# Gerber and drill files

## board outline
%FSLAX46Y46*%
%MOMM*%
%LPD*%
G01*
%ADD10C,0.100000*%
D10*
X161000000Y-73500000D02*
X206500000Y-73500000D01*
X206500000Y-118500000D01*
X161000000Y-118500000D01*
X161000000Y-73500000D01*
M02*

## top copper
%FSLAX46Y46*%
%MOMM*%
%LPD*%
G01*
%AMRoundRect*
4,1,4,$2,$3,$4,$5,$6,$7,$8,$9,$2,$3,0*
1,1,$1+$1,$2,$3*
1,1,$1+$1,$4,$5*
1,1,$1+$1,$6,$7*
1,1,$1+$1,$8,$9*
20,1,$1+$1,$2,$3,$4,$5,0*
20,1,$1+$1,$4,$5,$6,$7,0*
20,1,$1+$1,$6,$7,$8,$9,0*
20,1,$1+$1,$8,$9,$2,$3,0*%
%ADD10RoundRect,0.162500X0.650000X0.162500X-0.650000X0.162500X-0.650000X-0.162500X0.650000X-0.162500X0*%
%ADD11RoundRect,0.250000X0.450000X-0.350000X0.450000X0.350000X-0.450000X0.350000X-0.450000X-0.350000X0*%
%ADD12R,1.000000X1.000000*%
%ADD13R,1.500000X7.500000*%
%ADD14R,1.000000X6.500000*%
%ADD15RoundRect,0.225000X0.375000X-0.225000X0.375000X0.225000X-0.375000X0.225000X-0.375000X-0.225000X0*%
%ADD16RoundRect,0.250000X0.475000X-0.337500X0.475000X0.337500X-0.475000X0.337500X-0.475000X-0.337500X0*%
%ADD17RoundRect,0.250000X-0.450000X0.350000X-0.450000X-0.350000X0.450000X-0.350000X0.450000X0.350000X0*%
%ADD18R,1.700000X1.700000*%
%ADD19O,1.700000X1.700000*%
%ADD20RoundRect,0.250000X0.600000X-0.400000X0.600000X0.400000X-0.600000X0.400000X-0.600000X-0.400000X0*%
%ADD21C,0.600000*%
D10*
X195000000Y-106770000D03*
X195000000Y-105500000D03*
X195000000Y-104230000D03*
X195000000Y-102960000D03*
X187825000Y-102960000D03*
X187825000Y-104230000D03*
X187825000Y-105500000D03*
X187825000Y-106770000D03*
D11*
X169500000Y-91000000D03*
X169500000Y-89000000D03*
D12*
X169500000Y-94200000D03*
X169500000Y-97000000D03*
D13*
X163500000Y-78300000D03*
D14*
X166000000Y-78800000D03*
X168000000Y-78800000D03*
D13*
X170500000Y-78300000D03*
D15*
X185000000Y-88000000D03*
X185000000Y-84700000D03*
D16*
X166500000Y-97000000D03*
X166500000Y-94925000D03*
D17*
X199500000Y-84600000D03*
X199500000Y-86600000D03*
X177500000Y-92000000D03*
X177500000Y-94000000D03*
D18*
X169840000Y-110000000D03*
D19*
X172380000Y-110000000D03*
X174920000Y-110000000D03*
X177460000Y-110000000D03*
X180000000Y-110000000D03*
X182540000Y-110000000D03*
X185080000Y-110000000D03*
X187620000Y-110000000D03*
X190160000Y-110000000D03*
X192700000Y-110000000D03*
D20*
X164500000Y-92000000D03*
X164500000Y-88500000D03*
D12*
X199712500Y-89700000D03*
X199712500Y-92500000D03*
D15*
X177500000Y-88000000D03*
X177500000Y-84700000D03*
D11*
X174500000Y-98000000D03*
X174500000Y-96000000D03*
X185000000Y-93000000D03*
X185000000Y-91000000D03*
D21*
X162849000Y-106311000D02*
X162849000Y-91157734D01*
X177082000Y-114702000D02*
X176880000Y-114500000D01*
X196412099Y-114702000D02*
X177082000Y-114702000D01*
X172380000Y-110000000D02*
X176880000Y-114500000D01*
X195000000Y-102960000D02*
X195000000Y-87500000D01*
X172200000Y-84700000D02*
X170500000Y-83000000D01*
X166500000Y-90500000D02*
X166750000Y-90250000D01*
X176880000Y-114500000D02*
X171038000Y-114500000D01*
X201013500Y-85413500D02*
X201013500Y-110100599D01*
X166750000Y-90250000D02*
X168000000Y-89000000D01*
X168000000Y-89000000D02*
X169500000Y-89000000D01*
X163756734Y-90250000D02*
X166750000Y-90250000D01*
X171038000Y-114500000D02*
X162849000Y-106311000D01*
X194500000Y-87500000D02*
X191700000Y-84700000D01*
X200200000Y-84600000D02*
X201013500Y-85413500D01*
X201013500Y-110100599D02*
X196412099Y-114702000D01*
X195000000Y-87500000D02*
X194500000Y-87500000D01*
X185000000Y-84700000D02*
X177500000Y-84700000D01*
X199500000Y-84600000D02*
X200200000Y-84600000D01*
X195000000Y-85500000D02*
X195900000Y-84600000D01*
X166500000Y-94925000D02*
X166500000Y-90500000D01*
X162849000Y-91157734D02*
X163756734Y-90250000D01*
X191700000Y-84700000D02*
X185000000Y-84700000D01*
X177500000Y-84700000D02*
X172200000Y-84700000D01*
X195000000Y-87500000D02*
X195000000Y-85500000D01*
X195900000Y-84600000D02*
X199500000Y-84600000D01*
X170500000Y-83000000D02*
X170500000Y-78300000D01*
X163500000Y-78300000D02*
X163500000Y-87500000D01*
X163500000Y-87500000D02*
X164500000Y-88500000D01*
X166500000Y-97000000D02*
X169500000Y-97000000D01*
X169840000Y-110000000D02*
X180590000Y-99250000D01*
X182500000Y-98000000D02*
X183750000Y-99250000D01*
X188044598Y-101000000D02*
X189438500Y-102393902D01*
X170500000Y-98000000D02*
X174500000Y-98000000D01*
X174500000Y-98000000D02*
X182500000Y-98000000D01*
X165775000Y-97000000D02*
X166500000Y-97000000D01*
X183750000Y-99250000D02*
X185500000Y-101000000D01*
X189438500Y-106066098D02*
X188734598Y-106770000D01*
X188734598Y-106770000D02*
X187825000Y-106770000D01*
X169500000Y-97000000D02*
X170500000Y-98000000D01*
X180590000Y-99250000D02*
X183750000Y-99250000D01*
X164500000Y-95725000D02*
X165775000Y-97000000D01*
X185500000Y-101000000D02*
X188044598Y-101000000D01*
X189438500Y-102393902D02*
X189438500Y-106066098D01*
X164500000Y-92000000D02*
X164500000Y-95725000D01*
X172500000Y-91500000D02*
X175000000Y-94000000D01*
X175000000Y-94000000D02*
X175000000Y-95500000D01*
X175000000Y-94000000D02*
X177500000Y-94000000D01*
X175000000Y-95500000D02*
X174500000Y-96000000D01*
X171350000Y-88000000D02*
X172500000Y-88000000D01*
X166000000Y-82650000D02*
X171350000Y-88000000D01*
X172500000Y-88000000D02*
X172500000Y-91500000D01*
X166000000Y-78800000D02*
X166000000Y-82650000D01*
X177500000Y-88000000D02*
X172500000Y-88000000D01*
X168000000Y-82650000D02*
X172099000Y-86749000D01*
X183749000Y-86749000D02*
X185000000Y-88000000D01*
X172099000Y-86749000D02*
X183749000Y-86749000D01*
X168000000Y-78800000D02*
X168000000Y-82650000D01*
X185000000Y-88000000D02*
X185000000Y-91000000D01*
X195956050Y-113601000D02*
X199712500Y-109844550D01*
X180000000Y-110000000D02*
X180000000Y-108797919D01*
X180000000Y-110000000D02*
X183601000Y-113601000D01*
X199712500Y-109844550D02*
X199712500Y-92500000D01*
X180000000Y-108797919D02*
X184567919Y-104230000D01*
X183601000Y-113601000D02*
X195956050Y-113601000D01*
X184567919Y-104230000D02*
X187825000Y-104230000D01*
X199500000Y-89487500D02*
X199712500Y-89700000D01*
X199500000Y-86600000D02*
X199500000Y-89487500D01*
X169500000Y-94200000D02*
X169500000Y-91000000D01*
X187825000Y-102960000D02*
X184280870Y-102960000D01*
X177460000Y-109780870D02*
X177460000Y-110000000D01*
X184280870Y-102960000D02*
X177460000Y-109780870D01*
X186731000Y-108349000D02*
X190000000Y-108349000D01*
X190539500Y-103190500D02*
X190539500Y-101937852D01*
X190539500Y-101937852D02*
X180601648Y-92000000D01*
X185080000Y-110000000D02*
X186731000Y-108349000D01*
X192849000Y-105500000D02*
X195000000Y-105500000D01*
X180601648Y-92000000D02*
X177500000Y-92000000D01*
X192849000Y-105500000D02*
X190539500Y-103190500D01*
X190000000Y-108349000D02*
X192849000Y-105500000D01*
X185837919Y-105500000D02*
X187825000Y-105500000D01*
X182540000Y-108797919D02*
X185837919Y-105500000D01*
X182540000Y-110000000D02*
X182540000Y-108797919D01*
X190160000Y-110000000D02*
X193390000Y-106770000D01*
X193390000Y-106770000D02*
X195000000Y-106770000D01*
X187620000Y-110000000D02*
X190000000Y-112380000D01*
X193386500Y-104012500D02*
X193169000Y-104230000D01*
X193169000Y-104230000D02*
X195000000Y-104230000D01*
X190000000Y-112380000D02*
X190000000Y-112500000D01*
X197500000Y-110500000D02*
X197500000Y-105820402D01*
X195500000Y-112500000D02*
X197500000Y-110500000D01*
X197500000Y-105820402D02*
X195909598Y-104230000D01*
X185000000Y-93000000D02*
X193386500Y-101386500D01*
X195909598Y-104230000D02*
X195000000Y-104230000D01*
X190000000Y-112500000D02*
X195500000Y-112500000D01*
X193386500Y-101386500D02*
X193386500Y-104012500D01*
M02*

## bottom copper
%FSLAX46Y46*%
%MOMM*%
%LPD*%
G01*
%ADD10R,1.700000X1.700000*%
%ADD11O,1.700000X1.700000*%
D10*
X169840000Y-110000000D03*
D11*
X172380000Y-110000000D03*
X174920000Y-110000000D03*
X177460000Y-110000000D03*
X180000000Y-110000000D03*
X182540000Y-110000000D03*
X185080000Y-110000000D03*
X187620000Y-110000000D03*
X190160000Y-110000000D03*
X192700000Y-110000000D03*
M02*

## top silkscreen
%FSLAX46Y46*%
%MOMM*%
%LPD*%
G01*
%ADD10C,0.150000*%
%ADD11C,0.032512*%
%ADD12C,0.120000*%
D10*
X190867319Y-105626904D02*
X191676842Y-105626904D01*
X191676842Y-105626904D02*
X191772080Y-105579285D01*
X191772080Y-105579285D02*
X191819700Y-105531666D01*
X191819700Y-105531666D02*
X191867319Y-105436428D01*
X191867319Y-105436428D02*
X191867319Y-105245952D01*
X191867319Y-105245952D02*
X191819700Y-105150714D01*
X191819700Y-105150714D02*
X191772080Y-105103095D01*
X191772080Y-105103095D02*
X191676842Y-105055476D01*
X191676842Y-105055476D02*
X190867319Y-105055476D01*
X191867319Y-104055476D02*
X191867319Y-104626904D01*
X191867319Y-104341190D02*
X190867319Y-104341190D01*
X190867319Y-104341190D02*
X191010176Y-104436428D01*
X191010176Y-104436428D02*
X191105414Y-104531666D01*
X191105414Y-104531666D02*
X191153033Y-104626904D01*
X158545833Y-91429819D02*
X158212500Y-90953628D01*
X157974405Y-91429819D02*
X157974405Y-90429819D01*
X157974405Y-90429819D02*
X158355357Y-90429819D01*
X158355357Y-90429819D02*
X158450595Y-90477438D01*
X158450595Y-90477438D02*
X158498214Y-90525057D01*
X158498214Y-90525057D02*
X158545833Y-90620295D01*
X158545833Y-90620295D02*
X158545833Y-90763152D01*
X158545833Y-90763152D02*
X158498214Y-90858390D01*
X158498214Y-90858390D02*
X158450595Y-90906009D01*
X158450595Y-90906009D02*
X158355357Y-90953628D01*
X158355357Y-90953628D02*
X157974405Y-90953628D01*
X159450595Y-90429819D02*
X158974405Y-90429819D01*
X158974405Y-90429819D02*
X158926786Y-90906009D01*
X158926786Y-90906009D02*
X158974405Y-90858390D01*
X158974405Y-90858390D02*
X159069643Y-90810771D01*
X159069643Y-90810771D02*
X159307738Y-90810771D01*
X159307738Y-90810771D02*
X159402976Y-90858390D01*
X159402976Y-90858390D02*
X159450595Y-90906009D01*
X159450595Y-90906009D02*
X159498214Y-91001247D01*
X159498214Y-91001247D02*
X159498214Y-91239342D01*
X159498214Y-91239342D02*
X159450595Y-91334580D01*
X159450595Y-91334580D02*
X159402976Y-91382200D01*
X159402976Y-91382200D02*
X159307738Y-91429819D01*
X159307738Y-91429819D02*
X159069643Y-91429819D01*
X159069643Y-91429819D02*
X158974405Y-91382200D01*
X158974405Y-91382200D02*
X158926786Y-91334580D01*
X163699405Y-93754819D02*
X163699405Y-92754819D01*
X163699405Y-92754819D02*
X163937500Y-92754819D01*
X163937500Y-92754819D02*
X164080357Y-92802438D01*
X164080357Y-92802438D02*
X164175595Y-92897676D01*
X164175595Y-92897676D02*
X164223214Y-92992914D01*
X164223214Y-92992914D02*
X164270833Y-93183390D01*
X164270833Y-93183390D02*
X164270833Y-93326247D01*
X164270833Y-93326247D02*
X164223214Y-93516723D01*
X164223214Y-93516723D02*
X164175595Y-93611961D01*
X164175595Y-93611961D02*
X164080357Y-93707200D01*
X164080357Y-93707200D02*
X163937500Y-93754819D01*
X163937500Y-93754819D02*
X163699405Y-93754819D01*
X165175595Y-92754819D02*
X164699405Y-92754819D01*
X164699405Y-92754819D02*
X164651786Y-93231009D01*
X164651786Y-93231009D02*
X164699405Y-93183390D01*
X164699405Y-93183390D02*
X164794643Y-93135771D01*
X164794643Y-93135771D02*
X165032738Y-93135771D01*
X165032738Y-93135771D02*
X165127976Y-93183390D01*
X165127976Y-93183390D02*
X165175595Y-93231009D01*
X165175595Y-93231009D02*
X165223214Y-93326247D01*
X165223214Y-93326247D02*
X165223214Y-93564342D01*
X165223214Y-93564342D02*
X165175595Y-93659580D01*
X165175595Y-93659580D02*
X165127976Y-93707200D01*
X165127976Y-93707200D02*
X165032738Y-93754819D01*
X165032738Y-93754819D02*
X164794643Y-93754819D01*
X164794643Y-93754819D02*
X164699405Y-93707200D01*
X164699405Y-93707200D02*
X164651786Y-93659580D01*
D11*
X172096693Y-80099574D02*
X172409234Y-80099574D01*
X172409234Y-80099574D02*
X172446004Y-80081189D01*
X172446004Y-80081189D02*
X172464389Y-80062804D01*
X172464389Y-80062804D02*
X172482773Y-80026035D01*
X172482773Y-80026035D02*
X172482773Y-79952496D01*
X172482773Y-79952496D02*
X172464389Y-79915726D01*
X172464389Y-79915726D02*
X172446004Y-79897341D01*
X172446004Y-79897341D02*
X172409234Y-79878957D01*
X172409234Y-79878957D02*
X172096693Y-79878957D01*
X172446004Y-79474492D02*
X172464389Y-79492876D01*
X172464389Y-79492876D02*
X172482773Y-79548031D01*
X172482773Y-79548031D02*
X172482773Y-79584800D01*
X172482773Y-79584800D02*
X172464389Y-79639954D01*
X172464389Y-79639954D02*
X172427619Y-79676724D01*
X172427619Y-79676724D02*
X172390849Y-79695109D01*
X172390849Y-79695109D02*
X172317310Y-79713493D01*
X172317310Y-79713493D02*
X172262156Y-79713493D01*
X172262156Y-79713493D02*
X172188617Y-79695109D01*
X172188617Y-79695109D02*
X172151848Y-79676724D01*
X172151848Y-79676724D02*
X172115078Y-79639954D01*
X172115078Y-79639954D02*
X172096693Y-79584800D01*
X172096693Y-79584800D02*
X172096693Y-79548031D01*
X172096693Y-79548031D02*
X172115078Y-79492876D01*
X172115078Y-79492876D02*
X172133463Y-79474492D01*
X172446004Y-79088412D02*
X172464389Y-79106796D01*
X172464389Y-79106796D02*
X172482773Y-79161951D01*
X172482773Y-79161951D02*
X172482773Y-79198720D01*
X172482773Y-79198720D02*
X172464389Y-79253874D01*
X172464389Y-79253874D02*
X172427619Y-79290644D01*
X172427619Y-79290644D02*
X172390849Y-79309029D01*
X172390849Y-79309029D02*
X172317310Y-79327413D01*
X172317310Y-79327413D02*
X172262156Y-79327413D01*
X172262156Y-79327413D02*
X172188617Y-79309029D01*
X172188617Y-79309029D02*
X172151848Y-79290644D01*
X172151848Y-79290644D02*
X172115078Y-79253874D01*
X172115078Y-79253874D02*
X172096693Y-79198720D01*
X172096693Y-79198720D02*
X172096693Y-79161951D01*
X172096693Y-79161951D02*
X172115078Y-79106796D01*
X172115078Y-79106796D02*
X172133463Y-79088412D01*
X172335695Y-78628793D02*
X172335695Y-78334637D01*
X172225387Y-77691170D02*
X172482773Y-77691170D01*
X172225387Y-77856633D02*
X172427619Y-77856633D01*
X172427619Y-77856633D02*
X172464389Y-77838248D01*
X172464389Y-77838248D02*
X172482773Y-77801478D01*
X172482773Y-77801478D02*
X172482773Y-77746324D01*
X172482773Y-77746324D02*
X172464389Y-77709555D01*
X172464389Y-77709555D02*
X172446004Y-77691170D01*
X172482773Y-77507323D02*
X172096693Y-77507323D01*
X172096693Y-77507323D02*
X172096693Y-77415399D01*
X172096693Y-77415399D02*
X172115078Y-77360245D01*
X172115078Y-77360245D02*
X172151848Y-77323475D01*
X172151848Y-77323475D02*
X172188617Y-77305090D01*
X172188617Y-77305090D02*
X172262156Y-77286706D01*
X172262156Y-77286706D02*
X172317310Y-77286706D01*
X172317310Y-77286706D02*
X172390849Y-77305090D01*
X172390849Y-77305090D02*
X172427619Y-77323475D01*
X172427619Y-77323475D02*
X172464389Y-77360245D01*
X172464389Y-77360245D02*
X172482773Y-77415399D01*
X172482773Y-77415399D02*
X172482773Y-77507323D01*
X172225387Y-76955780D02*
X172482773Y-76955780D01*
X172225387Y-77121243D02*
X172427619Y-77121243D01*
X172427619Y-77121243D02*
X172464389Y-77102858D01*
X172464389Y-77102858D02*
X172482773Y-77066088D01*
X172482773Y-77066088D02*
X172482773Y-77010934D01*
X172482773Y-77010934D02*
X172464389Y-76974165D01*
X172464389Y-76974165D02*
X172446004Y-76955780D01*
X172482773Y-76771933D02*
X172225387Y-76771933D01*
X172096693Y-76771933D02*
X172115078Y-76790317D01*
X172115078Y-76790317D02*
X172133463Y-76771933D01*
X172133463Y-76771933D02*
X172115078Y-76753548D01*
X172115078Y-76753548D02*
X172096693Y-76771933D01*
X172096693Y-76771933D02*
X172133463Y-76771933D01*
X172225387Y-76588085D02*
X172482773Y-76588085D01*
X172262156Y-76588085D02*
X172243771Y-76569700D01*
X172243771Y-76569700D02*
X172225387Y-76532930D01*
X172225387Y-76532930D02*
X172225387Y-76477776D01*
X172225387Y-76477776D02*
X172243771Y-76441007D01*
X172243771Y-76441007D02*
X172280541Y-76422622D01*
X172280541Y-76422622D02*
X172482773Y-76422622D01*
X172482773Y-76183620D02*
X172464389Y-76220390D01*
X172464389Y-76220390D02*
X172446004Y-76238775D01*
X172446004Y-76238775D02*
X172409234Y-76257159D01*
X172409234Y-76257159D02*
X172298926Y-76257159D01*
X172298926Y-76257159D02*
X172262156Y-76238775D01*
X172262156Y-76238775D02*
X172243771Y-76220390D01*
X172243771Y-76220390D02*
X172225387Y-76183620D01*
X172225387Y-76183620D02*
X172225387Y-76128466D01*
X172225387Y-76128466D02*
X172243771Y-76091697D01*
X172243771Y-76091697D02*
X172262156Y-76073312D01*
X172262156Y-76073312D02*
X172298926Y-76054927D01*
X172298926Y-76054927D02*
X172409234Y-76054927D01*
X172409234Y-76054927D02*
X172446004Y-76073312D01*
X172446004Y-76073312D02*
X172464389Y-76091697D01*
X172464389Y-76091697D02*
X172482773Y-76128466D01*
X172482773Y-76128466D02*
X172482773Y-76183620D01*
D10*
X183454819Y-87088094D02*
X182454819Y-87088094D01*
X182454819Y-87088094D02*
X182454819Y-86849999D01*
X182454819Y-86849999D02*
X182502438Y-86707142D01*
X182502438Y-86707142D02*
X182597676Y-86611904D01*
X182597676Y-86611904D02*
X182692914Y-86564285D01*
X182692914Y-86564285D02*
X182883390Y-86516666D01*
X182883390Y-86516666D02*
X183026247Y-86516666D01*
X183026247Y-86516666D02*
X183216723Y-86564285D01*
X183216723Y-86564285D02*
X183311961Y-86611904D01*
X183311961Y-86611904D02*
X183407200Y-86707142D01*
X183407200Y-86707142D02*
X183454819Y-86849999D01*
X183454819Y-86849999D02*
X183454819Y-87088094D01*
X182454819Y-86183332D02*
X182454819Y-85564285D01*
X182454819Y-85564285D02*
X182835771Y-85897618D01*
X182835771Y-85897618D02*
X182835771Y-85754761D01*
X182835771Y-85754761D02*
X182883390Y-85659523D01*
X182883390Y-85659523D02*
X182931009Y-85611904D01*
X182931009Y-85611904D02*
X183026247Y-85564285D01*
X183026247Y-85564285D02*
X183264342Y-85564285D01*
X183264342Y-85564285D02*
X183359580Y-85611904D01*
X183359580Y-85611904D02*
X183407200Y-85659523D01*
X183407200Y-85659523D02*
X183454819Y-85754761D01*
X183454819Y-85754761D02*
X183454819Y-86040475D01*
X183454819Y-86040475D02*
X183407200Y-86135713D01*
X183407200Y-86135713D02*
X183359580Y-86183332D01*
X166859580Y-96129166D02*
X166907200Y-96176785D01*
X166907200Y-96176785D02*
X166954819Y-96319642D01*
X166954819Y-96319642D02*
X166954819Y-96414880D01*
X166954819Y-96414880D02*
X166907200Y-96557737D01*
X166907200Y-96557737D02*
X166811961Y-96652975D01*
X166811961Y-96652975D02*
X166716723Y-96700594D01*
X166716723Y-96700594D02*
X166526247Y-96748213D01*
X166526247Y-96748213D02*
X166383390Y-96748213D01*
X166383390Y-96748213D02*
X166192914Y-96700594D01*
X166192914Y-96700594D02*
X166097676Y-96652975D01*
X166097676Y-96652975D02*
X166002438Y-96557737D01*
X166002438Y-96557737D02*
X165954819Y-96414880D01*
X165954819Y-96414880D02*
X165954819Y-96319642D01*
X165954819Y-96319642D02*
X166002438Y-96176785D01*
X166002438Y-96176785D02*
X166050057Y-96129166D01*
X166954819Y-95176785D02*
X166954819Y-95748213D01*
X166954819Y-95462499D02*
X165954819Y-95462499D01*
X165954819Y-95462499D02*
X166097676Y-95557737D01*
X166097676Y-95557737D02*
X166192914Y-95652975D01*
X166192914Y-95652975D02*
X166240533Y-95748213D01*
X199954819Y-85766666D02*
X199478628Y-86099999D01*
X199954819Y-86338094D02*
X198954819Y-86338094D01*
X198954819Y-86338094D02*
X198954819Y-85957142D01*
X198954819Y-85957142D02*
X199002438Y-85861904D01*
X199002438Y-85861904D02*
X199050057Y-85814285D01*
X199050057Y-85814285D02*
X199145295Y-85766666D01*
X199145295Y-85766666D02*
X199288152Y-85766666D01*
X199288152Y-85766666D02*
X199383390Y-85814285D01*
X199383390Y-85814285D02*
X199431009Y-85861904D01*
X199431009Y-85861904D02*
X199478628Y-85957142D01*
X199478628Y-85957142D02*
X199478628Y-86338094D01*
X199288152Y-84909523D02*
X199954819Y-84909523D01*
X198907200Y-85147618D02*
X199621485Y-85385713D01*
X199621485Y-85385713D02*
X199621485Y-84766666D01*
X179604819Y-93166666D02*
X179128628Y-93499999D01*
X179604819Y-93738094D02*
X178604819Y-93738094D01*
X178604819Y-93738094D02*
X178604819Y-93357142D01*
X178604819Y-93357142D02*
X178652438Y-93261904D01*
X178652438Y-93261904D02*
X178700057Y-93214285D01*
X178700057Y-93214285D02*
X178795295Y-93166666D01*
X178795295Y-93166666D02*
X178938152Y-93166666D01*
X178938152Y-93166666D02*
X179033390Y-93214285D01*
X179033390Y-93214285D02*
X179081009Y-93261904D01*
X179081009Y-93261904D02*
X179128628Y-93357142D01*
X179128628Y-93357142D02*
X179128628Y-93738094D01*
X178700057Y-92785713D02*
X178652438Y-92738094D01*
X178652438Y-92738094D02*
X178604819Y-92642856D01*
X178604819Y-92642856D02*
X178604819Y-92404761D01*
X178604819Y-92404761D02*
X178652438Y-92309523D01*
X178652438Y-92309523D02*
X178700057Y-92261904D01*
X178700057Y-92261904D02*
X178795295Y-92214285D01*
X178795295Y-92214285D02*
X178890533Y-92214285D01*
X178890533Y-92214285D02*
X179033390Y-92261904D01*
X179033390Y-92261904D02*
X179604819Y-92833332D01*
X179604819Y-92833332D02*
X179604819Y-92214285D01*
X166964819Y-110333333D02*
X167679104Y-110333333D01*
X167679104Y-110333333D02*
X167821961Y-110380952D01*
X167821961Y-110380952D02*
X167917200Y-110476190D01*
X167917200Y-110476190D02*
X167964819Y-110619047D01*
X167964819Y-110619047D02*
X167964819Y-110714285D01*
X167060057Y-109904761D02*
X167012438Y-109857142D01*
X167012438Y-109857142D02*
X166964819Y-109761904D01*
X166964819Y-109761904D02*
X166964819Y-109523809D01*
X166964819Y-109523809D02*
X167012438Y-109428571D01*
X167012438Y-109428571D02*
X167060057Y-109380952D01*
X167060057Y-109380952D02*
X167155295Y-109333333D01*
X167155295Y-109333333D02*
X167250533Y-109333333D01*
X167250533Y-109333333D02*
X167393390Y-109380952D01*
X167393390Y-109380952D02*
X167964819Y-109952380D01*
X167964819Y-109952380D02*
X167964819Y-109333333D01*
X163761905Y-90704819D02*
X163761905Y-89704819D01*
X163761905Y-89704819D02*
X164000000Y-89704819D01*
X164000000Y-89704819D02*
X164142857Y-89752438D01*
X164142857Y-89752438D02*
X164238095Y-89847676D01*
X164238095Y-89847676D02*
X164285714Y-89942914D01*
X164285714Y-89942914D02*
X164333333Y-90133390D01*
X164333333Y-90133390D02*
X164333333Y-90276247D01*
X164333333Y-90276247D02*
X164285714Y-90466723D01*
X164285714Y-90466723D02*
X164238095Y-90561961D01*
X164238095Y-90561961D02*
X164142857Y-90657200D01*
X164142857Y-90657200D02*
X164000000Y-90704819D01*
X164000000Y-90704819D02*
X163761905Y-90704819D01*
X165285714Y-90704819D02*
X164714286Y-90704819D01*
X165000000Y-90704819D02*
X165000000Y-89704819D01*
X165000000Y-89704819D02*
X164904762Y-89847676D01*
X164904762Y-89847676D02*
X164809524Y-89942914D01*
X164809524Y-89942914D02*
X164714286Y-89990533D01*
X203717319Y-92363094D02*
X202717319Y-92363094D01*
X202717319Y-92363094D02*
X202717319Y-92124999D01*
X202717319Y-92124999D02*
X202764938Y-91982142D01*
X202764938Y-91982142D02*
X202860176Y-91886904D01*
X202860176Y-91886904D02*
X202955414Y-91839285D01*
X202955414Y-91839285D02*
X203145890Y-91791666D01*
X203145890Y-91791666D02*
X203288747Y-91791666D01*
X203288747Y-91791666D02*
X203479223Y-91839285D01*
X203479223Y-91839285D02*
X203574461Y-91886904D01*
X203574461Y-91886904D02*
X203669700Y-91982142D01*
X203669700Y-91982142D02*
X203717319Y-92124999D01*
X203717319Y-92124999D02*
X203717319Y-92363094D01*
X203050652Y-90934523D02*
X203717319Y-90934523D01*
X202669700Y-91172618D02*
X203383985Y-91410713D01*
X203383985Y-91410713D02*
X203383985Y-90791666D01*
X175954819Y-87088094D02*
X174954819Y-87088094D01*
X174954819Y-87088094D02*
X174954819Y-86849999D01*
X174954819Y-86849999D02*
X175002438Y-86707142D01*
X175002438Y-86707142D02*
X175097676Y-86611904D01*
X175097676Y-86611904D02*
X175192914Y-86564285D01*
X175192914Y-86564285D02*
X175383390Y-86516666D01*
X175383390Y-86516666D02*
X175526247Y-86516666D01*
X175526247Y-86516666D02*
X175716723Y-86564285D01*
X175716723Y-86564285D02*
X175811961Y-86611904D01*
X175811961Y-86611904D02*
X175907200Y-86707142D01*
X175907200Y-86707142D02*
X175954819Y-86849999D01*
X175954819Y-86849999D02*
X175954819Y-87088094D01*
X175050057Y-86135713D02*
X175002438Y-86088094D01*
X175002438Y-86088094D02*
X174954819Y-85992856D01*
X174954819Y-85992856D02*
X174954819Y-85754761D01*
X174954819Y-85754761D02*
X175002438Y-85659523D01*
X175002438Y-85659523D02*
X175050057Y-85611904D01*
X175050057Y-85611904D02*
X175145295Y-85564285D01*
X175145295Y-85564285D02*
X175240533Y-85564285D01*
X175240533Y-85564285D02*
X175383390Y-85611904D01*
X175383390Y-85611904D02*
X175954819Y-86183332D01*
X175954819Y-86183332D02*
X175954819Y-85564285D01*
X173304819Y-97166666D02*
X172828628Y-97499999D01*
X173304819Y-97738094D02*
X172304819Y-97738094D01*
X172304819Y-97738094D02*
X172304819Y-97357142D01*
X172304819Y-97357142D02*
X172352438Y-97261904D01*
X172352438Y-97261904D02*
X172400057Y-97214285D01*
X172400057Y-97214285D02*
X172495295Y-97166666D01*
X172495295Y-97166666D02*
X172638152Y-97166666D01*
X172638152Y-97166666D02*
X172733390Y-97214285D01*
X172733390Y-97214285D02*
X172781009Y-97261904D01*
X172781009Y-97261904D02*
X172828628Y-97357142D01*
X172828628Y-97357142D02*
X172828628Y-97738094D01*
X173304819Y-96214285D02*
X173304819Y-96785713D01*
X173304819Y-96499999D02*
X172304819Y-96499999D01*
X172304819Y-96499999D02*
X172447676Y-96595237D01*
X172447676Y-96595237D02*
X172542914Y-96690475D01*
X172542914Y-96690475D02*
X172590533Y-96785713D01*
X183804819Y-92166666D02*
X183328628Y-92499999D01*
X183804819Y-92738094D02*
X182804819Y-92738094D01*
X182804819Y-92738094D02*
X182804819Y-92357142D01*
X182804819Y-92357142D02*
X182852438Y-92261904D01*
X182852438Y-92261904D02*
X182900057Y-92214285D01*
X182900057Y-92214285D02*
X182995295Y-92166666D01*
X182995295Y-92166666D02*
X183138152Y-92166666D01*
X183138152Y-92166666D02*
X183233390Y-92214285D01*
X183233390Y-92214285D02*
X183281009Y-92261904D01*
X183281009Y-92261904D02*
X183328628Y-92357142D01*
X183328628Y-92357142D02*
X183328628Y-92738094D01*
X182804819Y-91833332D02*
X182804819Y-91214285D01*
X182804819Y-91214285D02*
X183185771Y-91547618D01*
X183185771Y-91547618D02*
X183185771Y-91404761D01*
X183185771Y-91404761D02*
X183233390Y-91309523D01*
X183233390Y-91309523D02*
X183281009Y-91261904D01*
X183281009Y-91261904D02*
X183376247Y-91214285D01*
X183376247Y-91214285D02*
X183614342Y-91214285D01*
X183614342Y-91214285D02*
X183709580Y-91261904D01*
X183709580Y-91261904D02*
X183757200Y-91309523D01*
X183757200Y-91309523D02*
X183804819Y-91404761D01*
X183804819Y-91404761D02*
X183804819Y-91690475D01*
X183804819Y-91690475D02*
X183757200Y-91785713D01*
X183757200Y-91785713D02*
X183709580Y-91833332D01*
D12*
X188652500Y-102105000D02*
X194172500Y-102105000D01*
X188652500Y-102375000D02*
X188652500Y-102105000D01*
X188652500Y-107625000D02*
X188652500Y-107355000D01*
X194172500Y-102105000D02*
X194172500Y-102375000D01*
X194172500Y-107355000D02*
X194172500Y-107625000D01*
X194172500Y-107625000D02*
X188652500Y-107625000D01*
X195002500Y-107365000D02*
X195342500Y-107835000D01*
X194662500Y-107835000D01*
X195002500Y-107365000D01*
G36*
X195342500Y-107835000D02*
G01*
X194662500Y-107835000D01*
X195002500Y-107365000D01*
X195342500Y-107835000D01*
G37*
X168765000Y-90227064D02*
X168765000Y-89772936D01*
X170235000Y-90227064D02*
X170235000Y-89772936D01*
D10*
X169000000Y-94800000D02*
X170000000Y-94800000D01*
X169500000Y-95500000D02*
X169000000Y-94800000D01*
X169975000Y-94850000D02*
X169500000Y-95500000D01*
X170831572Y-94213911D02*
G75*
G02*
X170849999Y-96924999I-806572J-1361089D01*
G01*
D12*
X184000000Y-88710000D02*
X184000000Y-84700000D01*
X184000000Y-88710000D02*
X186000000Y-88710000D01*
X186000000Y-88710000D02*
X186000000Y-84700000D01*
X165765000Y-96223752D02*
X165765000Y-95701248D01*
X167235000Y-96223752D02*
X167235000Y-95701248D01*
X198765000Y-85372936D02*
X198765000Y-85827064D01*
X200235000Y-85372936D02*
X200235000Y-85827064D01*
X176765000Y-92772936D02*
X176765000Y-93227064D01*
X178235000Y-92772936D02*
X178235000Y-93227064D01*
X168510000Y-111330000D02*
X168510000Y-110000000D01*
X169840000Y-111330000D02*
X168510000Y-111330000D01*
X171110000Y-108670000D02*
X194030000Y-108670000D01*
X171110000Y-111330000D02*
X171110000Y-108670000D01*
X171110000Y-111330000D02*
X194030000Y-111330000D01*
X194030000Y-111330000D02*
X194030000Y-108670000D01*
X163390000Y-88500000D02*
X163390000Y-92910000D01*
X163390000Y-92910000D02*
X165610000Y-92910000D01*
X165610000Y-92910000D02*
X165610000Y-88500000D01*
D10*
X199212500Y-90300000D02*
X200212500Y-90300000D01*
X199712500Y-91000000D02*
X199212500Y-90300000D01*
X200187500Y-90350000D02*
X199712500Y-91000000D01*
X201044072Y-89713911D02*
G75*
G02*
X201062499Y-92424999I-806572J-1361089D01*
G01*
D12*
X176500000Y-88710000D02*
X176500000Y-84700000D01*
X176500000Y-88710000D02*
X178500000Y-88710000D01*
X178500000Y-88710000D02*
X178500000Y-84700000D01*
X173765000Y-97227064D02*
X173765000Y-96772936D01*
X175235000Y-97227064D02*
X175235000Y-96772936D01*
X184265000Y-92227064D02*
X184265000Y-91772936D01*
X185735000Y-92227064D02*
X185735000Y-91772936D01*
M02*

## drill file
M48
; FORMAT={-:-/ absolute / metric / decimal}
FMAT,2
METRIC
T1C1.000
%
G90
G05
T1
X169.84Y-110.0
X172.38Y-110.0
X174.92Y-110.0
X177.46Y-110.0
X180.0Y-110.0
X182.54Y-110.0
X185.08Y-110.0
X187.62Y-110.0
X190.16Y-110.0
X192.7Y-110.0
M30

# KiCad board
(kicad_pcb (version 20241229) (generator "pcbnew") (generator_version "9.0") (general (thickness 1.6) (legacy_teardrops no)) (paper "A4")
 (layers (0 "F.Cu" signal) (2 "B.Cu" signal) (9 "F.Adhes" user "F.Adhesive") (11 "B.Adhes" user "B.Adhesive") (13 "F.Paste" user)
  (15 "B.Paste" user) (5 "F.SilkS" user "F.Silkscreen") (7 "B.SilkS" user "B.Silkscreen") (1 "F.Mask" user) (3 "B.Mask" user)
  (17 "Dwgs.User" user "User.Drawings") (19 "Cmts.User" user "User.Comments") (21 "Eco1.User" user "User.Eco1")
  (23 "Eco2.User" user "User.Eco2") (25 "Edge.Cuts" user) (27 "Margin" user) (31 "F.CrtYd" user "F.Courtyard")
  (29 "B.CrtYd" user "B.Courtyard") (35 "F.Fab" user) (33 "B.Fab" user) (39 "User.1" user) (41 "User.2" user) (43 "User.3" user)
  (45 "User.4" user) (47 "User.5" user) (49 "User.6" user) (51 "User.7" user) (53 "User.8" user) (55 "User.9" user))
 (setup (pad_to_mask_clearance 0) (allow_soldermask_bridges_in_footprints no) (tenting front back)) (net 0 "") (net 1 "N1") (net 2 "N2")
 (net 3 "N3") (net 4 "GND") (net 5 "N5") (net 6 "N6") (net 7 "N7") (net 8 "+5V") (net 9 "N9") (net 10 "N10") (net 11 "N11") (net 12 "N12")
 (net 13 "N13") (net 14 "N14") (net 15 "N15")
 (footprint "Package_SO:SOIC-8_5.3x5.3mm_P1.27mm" (layer "F.Cu") (at 191.4125 104.865 180)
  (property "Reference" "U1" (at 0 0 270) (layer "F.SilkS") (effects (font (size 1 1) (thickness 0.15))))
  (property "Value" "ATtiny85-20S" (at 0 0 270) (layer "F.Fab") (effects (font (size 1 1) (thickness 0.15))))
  (fp_line (start 2.76 2.76) (end -2.76 2.76) (stroke (width 0.12) (type solid)) (layer "F.SilkS"))
  (fp_line (start 2.76 2.49) (end 2.76 2.76) (stroke (width 0.12) (type solid)) (layer "F.SilkS"))
  (fp_line (start 2.76 -2.76) (end 2.76 -2.49) (stroke (width 0.12) (type solid)) (layer "F.SilkS"))
  (fp_line (start -2.76 2.76) (end -2.76 2.49) (stroke (width 0.12) (type solid)) (layer "F.SilkS"))
  (fp_line (start -2.76 -2.49) (end -2.76 -2.76) (stroke (width 0.12) (type solid)) (layer "F.SilkS"))
  (fp_line (start -2.76 -2.76) (end 2.76 -2.76) (stroke (width 0.12) (type solid)) (layer "F.SilkS"))
  (fp_poly (pts (xy -3.59 -2.5) (xy -3.93 -2.97) (xy -3.25 -2.97)) (stroke (width 0.12) (type solid)) (fill yes) (layer "F.SilkS"))
  (pad "1" smd roundrect (at -3.5875 -1.905 180) (size 1.625 0.65) (layers "F.Cu" "F.Mask" "F.Paste") (roundrect_rratio 0.25) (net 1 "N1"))
  (pad "2" smd roundrect (at -3.5875 -0.635 180) (size 1.625 0.65) (layers "F.Cu" "F.Mask" "F.Paste") (roundrect_rratio 0.25) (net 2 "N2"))
  (pad "3" smd roundrect (at -3.5875 0.635 180) (size 1.625 0.65) (layers "F.Cu" "F.Mask" "F.Paste") (roundrect_rratio 0.25) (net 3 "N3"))
  (pad "4" smd roundrect (at -3.5875 1.905 180) (size 1.625 0.65) (layers "F.Cu" "F.Mask" "F.Paste") (roundrect_rratio 0.25) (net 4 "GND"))
  (pad "5" smd roundrect (at 3.5875 1.905 180) (size 1.625 0.65) (layers "F.Cu" "F.Mask" "F.Paste") (roundrect_rratio 0.25) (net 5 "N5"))
  (pad "6" smd roundrect (at 3.5875 0.635 180) (size 1.625 0.65) (layers "F.Cu" "F.Mask" "F.Paste") (roundrect_rratio 0.25) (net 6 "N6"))
  (pad "7" smd roundrect (at 3.5875 -0.635 180) (size 1.625 0.65) (layers "F.Cu" "F.Mask" "F.Paste") (roundrect_rratio 0.25) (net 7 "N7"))
  (pad "8" smd roundrect (at 3.5875 -1.905 180) (size 1.625 0.65) (layers "F.Cu" "F.Mask" "F.Paste") (roundrect_rratio 0.25) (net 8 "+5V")))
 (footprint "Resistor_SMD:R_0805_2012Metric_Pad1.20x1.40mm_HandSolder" (layer "F.Cu") (at 169.5 90 90)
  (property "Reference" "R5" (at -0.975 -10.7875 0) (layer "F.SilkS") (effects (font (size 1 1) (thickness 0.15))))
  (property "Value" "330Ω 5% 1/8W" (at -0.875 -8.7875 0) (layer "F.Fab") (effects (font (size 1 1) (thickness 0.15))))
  (fp_line (start -0.227064 -0.735) (end 0.227064 -0.735) (stroke (width 0.12) (type solid)) (layer "F.SilkS"))
  (fp_line (start -0.227064 0.735) (end 0.227064 0.735) (stroke (width 0.12) (type solid)) (layer "F.SilkS"))
  (pad "1" smd roundrect (at -1 0 90) (size 1.2 1.4) (layers "F.Cu" "F.Mask" "F.Paste") (roundrect_rratio 0.208333) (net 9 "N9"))
  (pad "2" smd roundrect (at 1 0 90) (size 1.2 1.4) (layers "F.Cu" "F.Mask" "F.Paste") (roundrect_rratio 0.208333) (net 4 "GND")))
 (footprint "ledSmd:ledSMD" (layer "F.Cu") (at 169.5 96 -90)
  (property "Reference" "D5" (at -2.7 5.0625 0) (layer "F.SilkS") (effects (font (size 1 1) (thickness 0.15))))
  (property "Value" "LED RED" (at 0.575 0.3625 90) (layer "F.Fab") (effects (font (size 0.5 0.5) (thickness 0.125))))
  (fp_line (start -1.2 0.5) (end -1.2 -0.5) (stroke (width 0.15) (type solid)) (layer "F.SilkS"))
  (fp_line (start -0.5 0) (end -1.2 0.5) (stroke (width 0.15) (type solid)) (layer "F.SilkS"))
  (fp_line (start -1.15 -0.475) (end -0.5 0) (stroke (width 0.15) (type solid)) (layer "F.SilkS"))
  (fp_arc (start -1.786089 -1.331572) (mid -0.435753 -2.107089) (end 0.924999 -1.349999) (stroke (width 0.15) (type solid))
   (layer "F.SilkS"))
  (pad "1" smd rect (at -1.8 0 270) (size 1 1) (layers "F.Cu" "F.Mask" "F.Paste") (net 9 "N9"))
  (pad "2" smd rect (at 1 0 270) (size 1 1) (layers "F.Cu" "F.Mask" "F.Paste") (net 8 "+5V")))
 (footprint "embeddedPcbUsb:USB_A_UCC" (layer "F.Cu") (at 167 78.5 -90)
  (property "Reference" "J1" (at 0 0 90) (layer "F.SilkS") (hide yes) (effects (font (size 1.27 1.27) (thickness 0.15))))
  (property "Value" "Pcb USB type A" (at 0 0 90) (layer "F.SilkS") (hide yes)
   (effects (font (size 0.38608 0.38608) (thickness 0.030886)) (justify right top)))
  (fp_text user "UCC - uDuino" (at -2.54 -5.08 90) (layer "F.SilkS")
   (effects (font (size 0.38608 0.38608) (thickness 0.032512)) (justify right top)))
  (pad "1" smd rect (at -0.2 3.5 270) (size 7.5 1.5) (layers "F.Cu" "F.Mask" "F.Paste") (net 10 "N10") (solder_mask_margin 0.1016))
  (pad "2" smd rect (at 0.3 1 270) (size 6.5 1) (layers "F.Cu" "F.Mask" "F.Paste") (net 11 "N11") (solder_mask_margin 0.1016))
  (pad "3" smd rect (at 0.3 -1 270) (size 6.5 1) (layers "F.Cu" "F.Mask" "F.Paste") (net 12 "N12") (solder_mask_margin 0.1016))
  (pad "4" smd rect (at -0.2 -3.5 270) (size 7.5 1.5) (layers "F.Cu" "F.Mask" "F.Paste") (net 4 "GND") (solder_mask_margin 0.1016)))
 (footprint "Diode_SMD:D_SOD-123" (layer "F.Cu") (at 185 86.35 90)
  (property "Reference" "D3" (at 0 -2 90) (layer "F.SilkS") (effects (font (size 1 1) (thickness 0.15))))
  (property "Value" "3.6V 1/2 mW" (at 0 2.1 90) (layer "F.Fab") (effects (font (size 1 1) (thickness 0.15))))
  (fp_line (start -2.36 -1) (end 1.65 -1) (stroke (width 0.12) (type solid)) (layer "F.SilkS"))
  (fp_line (start -2.36 -1) (end -2.36 1) (stroke (width 0.12) (type solid)) (layer "F.SilkS"))
  (fp_line (start -2.36 1) (end 1.65 1) (stroke (width 0.12) (type solid)) (layer "F.SilkS"))
  (pad "1" smd roundrect (at -1.65 0 90) (size 0.9 1.2) (layers "F.Cu" "F.Mask" "F.Paste") (roundrect_rratio 0.25) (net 12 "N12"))
  (pad "2" smd roundrect (at 1.65 0 90) (size 0.9 1.2) (layers "F.Cu" "F.Mask" "F.Paste") (roundrect_rratio 0.25) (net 4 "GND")))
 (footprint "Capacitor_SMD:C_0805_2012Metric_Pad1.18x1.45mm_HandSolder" (layer "F.Cu") (at 166.5 95.9625 90)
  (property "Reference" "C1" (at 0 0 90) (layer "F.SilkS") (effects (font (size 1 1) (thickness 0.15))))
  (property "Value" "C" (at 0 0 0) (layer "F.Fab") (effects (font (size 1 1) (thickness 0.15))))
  (fp_line (start -0.261252 -0.735) (end 0.261252 -0.735) (stroke (width 0.12) (type solid)) (layer "F.SilkS"))
  (fp_line (start -0.261252 0.735) (end 0.261252 0.735) (stroke (width 0.12) (type solid)) (layer "F.SilkS"))
  (pad "1" smd roundrect (at -1.0375 0 90) (size 1.175 1.45) (layers "F.Cu" "F.Mask" "F.Paste") (roundrect_rratio 0.212766) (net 8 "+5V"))
  (pad "2" smd roundrect (at 1.0375 0 90) (size 1.175 1.45) (layers "F.Cu" "F.Mask" "F.Paste") (roundrect_rratio 0.212766) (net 4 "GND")))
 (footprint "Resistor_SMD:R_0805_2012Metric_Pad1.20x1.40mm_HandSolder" (layer "F.Cu") (at 199.5 85.6 -90)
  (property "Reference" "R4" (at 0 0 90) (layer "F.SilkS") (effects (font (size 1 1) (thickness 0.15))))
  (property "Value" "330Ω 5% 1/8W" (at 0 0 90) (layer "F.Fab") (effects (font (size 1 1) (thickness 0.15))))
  (fp_line (start -0.227064 0.735) (end 0.227064 0.735) (stroke (width 0.12) (type solid)) (layer "F.SilkS"))
  (fp_line (start -0.227064 -0.735) (end 0.227064 -0.735) (stroke (width 0.12) (type solid)) (layer "F.SilkS"))
  (pad "1" smd roundrect (at -1 0 270) (size 1.2 1.4) (layers "F.Cu" "F.Mask" "F.Paste") (roundrect_rratio 0.208333) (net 4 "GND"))
  (pad "2" smd roundrect (at 1 0 270) (size 1.2 1.4) (layers "F.Cu" "F.Mask" "F.Paste") (roundrect_rratio 0.208333) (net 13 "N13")))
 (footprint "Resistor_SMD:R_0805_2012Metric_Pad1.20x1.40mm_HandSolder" (layer "F.Cu") (at 177.5 93 -90)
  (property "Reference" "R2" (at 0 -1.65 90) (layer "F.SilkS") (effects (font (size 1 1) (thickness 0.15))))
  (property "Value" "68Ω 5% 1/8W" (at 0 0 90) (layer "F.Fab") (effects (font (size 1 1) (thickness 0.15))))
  (fp_line (start -0.227064 0.735) (end 0.227064 0.735) (stroke (width 0.12) (type solid)) (layer "F.SilkS"))
  (fp_line (start -0.227064 -0.735) (end 0.227064 -0.735) (stroke (width 0.12) (type solid)) (layer "F.SilkS"))
  (pad "1" smd roundrect (at -1 0 270) (size 1.2 1.4) (layers "F.Cu" "F.Mask" "F.Paste") (roundrect_rratio 0.208333) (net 2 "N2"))
  (pad "2" smd roundrect (at 1 0 270) (size 1.2 1.4) (layers "F.Cu" "F.Mask" "F.Paste") (roundrect_rratio 0.208333) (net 11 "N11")))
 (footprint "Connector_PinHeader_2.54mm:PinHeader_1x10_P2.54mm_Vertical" (layer "F.Cu") (at 169.84 110 90)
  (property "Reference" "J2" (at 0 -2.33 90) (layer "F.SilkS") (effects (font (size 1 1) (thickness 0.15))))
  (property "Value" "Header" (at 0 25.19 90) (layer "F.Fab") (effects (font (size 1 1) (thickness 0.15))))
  (fp_line (start -1.33 -1.33) (end 0 -1.33) (stroke (width 0.12) (type solid)) (layer "F.SilkS"))
  (fp_line (start -1.33 0) (end -1.33 -1.33) (stroke (width 0.12) (type solid)) (layer "F.SilkS"))
  (fp_line (start 1.33 1.27) (end 1.33 24.19) (stroke (width 0.12) (type solid)) (layer "F.SilkS"))
  (fp_line (start -1.33 1.27) (end 1.33 1.27) (stroke (width 0.12) (type solid)) (layer "F.SilkS"))
  (fp_line (start -1.33 1.27) (end -1.33 24.19) (stroke (width 0.12) (type solid)) (layer "F.SilkS"))
  (fp_line (start -1.33 24.19) (end 1.33 24.19) (stroke (width 0.12) (type solid)) (layer "F.SilkS"))
  (pad "1" thru_hole rect (at 0 0 90) (size 1.7 1.7) (drill 1) (layers "*.Cu" "*.Mask") (remove_unused_layers no) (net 8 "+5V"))
  (pad "2" thru_hole oval (at 0 2.54 90) (size 1.7 1.7) (drill 1) (layers "*.Cu" "*.Mask") (remove_unused_layers no) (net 4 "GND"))
  (pad "3" thru_hole oval (at 0 5.08 90) (size 1.7 1.7) (drill 1) (layers "*.Cu" "*.Mask") (remove_unused_layers no) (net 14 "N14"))
  (pad "4" thru_hole oval (at 0 7.62 90) (size 1.7 1.7) (drill 1) (layers "*.Cu" "*.Mask") (remove_unused_layers no) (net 5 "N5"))
  (pad "5" thru_hole oval (at 0 10.16 90) (size 1.7 1.7) (drill 1) (layers "*.Cu" "*.Mask") (remove_unused_layers no) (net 6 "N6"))
  (pad "6" thru_hole oval (at 0 12.7 90) (size 1.7 1.7) (drill 1) (layers "*.Cu" "*.Mask") (remove_unused_layers no) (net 7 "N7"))
  (pad "7" thru_hole oval (at 0 15.24 90) (size 1.7 1.7) (drill 1) (layers "*.Cu" "*.Mask") (remove_unused_layers no) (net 2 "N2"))
  (pad "8" thru_hole oval (at 0 17.78 90) (size 1.7 1.7) (drill 1) (layers "*.Cu" "*.Mask") (remove_unused_layers no) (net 3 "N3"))
  (pad "9" thru_hole oval (at 0 20.32 90) (size 1.7 1.7) (drill 1) (layers "*.Cu" "*.Mask") (remove_unused_layers no) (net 1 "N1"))
  (pad "10" thru_hole oval (at 0 22.86 90) (size 1.7 1.7) (drill 1) (layers "*.Cu" "*.Mask") (remove_unused_layers no) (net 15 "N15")))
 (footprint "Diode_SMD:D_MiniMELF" (layer "F.Cu") (at 164.5 90.25 90)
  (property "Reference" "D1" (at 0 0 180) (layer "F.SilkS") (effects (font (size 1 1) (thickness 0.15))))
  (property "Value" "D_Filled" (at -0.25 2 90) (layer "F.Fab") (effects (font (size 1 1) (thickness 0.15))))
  (fp_line (start 1.75 -1.11) (end -2.66 -1.11) (stroke (width 0.12) (type solid)) (layer "F.SilkS"))
  (fp_line (start -2.66 -1.11) (end -2.66 1.11) (stroke (width 0.12) (type solid)) (layer "F.SilkS"))
  (fp_line (start -2.66 1.11) (end 1.75 1.11) (stroke (width 0.12) (type solid)) (layer "F.SilkS"))
  (pad "1" smd roundrect (at -1.75 0 90) (size 1.3 1.7) (layers "F.Cu" "F.Mask" "F.Paste") (roundrect_rratio 0.1923076923) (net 8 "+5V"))
  (pad "2" smd roundrect (at 1.75 0 90) (size 1.3 1.7) (layers "F.Cu" "F.Mask" "F.Paste") (roundrect_rratio 0.1923076923) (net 10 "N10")))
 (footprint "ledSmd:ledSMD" (layer "F.Cu") (at 199.7125 91.5 -90)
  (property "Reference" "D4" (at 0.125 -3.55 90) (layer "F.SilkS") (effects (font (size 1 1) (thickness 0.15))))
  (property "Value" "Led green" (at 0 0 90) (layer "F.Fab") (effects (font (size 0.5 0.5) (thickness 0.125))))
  (fp_line (start -1.2 0.5) (end -1.2 -0.5) (stroke (width 0.15) (type solid)) (layer "F.SilkS"))
  (fp_line (start -0.5 0) (end -1.2 0.5) (stroke (width 0.15) (type solid)) (layer "F.SilkS"))
  (fp_line (start -1.15 -0.475) (end -0.5 0) (stroke (width 0.15) (type solid)) (layer "F.SilkS"))
  (fp_arc (start -1.786089 -1.331572) (mid -0.435753 -2.107089) (end 0.924999 -1.349999) (stroke (width 0.15) (type solid))
   (layer "F.SilkS"))
  (pad "1" smd rect (at -1.8 0 270) (size 1 1) (layers "F.Cu" "F.Mask" "F.Paste") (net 13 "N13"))
  (pad "2" smd rect (at 1 0 270) (size 1 1) (layers "F.Cu" "F.Mask" "F.Paste") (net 6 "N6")))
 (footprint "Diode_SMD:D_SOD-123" (layer "F.Cu") (at 177.5 86.35 90)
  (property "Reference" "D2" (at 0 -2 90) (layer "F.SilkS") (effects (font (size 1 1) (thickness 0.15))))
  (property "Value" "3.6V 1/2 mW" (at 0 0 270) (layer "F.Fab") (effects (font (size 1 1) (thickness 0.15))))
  (fp_line (start -2.36 -1) (end 1.65 -1) (stroke (width 0.12) (type solid)) (layer "F.SilkS"))
  (fp_line (start -2.36 -1) (end -2.36 1) (stroke (width 0.12) (type solid)) (layer "F.SilkS"))
  (fp_line (start -2.36 1) (end 1.65 1) (stroke (width 0.12) (type solid)) (layer "F.SilkS"))
  (pad "1" smd roundrect (at -1.65 0 90) (size 0.9 1.2) (layers "F.Cu" "F.Mask" "F.Paste") (roundrect_rratio 0.25) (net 11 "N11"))
  (pad "2" smd roundrect (at 1.65 0 90) (size 0.9 1.2) (layers "F.Cu" "F.Mask" "F.Paste") (roundrect_rratio 0.25) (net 4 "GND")))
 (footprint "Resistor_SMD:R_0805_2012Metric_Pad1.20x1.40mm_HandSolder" (layer "F.Cu") (at 174.5 97 90)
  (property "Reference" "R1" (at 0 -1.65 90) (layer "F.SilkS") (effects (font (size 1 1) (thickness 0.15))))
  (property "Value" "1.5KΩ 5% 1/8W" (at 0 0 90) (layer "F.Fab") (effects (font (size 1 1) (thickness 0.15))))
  (fp_line (start -0.227064 -0.735) (end 0.227064 -0.735) (stroke (width 0.12) (type solid)) (layer "F.SilkS"))
  (fp_line (start -0.227064 0.735) (end 0.227064 0.735) (stroke (width 0.12) (type solid)) (layer "F.SilkS"))
  (pad "1" smd roundrect (at -1 0 90) (size 1.2 1.4) (layers "F.Cu" "F.Mask" "F.Paste") (roundrect_rratio 0.208333) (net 8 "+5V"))
  (pad "2" smd roundrect (at 1 0 90) (size 1.2 1.4) (layers "F.Cu" "F.Mask" "F.Paste") (roundrect_rratio 0.208333) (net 11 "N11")))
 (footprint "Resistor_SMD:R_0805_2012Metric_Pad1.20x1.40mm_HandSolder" (layer "F.Cu") (at 185 92 90)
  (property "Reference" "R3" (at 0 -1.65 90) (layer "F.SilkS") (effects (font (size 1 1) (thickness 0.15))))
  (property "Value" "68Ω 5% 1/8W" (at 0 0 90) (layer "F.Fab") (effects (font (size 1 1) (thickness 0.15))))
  (fp_line (start -0.227064 -0.735) (end 0.227064 -0.735) (stroke (width 0.12) (type solid)) (layer "F.SilkS"))
  (fp_line (start -0.227064 0.735) (end 0.227064 0.735) (stroke (width 0.12) (type solid)) (layer "F.SilkS"))
  (pad "1" smd roundrect (at -1 0 90) (size 1.2 1.4) (layers "F.Cu" "F.Mask" "F.Paste") (roundrect_rratio 0.208333) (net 3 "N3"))
  (pad "2" smd roundrect (at 1 0 90) (size 1.2 1.4) (layers "F.Cu" "F.Mask" "F.Paste") (roundrect_rratio 0.208333) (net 12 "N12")))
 (gr_rect (start 161 73.5) (end 206.5 118.5) (stroke (width 0.1) (type default)) (fill no) (layer "Edge.Cuts"))
 (segment (start 162.849 106.311) (end 162.849 91.157734) (width 0.6) (layer "F.Cu") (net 4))
 (segment (start 177.082 114.702) (end 176.88 114.5) (width 0.6) (layer "F.Cu") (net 4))
 (segment (start 196.412099 114.702) (end 177.082 114.702) (width 0.6) (layer "F.Cu") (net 4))
 (segment (start 172.38 110) (end 176.88 114.5) (width 0.6) (layer "F.Cu") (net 4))
 (segment (start 195 102.96) (end 195 87.5) (width 0.6) (layer "F.Cu") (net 4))
 (segment (start 172.2 84.7) (end 170.5 83) (width 0.6) (layer "F.Cu") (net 4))
 (segment (start 166.5 90.5) (end 166.75 90.25) (width 0.6) (layer "F.Cu") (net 4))
 (segment (start 176.88 114.5) (end 171.038 114.5) (width 0.6) (layer "F.Cu") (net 4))
 (segment (start 201.0135 85.4135) (end 201.0135 110.100599) (width 0.6) (layer "F.Cu") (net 4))
 (segment (start 166.75 90.25) (end 168 89) (width 0.6) (layer "F.Cu") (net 4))
 (segment (start 168 89) (end 169.5 89) (width 0.6) (layer "F.Cu") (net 4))
 (segment (start 163.756734 90.25) (end 166.75 90.25) (width 0.6) (layer "F.Cu") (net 4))
 (segment (start 171.038 114.5) (end 162.849 106.311) (width 0.6) (layer "F.Cu") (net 4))
 (segment (start 194.5 87.5) (end 191.7 84.7) (width 0.6) (layer "F.Cu") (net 4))
 (segment (start 200.2 84.6) (end 201.0135 85.4135) (width 0.6) (layer "F.Cu") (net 4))
 (segment (start 201.0135 110.100599) (end 196.412099 114.702) (width 0.6) (layer "F.Cu") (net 4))
 (segment (start 195 87.5) (end 194.5 87.5) (width 0.6) (layer "F.Cu") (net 4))
 (segment (start 185 84.7) (end 177.5 84.7) (width 0.6) (layer "F.Cu") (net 4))
 (segment (start 199.5 84.6) (end 200.2 84.6) (width 0.6) (layer "F.Cu") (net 4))
 (segment (start 195 85.5) (end 195.9 84.6) (width 0.6) (layer "F.Cu") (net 4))
 (segment (start 166.5 94.925) (end 166.5 90.5) (width 0.6) (layer "F.Cu") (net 4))
 (segment (start 162.849 91.157734) (end 163.756734 90.25) (width 0.6) (layer "F.Cu") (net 4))
 (segment (start 191.7 84.7) (end 185 84.7) (width 0.6) (layer "F.Cu") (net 4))
 (segment (start 177.5 84.7) (end 172.2 84.7) (width 0.6) (layer "F.Cu") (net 4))
 (segment (start 195 87.5) (end 195 85.5) (width 0.6) (layer "F.Cu") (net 4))
 (segment (start 195.9 84.6) (end 199.5 84.6) (width 0.6) (layer "F.Cu") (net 4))
 (segment (start 170.5 83) (end 170.5 78.3) (width 0.6) (layer "F.Cu") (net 4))
 (segment (start 163.5 78.3) (end 163.5 87.5) (width 0.6) (layer "F.Cu") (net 10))
 (segment (start 163.5 87.5) (end 164.5 88.5) (width 0.6) (layer "F.Cu") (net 10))
 (segment (start 166.5 97) (end 169.5 97) (width 0.6) (layer "F.Cu") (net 8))
 (segment (start 169.84 110) (end 180.59 99.25) (width 0.6) (layer "F.Cu") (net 8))
 (segment (start 182.5 98) (end 183.75 99.25) (width 0.6) (layer "F.Cu") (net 8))
 (segment (start 188.044598 101) (end 189.4385 102.393902) (width 0.6) (layer "F.Cu") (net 8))
 (segment (start 170.5 98) (end 174.5 98) (width 0.6) (layer "F.Cu") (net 8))
 (segment (start 174.5 98) (end 182.5 98) (width 0.6) (layer "F.Cu") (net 8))
 (segment (start 165.775 97) (end 166.5 97) (width 0.6) (layer "F.Cu") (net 8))
 (segment (start 183.75 99.25) (end 185.5 101) (width 0.6) (layer "F.Cu") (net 8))
 (segment (start 189.4385 106.066098) (end 188.734598 106.77) (width 0.6) (layer "F.Cu") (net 8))
 (segment (start 188.734598 106.77) (end 187.825 106.77) (width 0.6) (layer "F.Cu") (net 8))
 (segment (start 169.5 97) (end 170.5 98) (width 0.6) (layer "F.Cu") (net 8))
 (segment (start 180.59 99.25) (end 183.75 99.25) (width 0.6) (layer "F.Cu") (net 8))
 (segment (start 164.5 95.725) (end 165.775 97) (width 0.6) (layer "F.Cu") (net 8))
 (segment (start 185.5 101) (end 188.044598 101) (width 0.6) (layer "F.Cu") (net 8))
 (segment (start 189.4385 102.393902) (end 189.4385 106.066098) (width 0.6) (layer "F.Cu") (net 8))
 (segment (start 164.5 92) (end 164.5 95.725) (width 0.6) (layer "F.Cu") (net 8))
 (segment (start 172.5 91.5) (end 175 94) (width 0.6) (layer "F.Cu") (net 11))
 (segment (start 175 94) (end 175 95.5) (width 0.6) (layer "F.Cu") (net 11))
 (segment (start 175 94) (end 177.5 94) (width 0.6) (layer "F.Cu") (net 11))
 (segment (start 175 95.5) (end 174.5 96) (width 0.6) (layer "F.Cu") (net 11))
 (segment (start 171.35 88) (end 172.5 88) (width 0.6) (layer "F.Cu") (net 11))
 (segment (start 166 82.65) (end 171.35 88) (width 0.6) (layer "F.Cu") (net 11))
 (segment (start 172.5 88) (end 172.5 91.5) (width 0.6) (layer "F.Cu") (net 11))
 (segment (start 166 78.8) (end 166 82.65) (width 0.6) (layer "F.Cu") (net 11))
 (segment (start 177.5 88) (end 172.5 88) (width 0.6) (layer "F.Cu") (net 11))
 (segment (start 168 82.65) (end 172.099 86.749) (width 0.6) (layer "F.Cu") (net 12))
 (segment (start 183.749 86.749) (end 185 88) (width 0.6) (layer "F.Cu") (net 12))
 (segment (start 172.099 86.749) (end 183.749 86.749) (width 0.6) (layer "F.Cu") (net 12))
 (segment (start 168 78.8) (end 168 82.65) (width 0.6) (layer "F.Cu") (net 12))
 (segment (start 185 88) (end 185 91) (width 0.6) (layer "F.Cu") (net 12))
 (segment (start 195.95605 113.601) (end 199.7125 109.84455) (width 0.6) (layer "F.Cu") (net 6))
 (segment (start 180 110) (end 180 108.797919) (width 0.6) (layer "F.Cu") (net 6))
 (segment (start 180 110) (end 183.601 113.601) (width 0.6) (layer "F.Cu") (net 6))
 (segment (start 199.7125 109.84455) (end 199.7125 92.5) (width 0.6) (layer "F.Cu") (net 6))
 (segment (start 180 108.797919) (end 184.567919 104.23) (width 0.6) (layer "F.Cu") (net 6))
 (segment (start 183.601 113.601) (end 195.95605 113.601) (width 0.6) (layer "F.Cu") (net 6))
 (segment (start 184.567919 104.23) (end 187.825 104.23) (width 0.6) (layer "F.Cu") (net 6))
 (segment (start 199.5 89.4875) (end 199.7125 89.7) (width 0.6) (layer "F.Cu") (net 13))
 (segment (start 199.5 86.6) (end 199.5 89.4875) (width 0.6) (layer "F.Cu") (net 13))
 (segment (start 169.5 94.2) (end 169.5 91) (width 0.6) (layer "F.Cu") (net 9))
 (segment (start 187.825 102.96) (end 184.28087 102.96) (width 0.6) (layer "F.Cu") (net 5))
 (segment (start 177.46 109.78087) (end 177.46 110) (width 0.6) (layer "F.Cu") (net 5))
 (segment (start 184.28087 102.96) (end 177.46 109.78087) (width 0.6) (layer "F.Cu") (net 5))
 (segment (start 186.731 108.349) (end 190 108.349) (width 0.6) (layer "F.Cu") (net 2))
 (segment (start 190.5395 103.1905) (end 190.5395 101.937852) (width 0.6) (layer "F.Cu") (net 2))
 (segment (start 190.5395 101.937852) (end 180.601648 92) (width 0.6) (layer "F.Cu") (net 2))
 (segment (start 185.08 110) (end 186.731 108.349) (width 0.6) (layer "F.Cu") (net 2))
 (segment (start 192.849 105.5) (end 195 105.5) (width 0.6) (layer "F.Cu") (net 2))
 (segment (start 180.601648 92) (end 177.5 92) (width 0.6) (layer "F.Cu") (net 2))
 (segment (start 192.849 105.5) (end 190.5395 103.1905) (width 0.6) (layer "F.Cu") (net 2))
 (segment (start 190 108.349) (end 192.849 105.5) (width 0.6) (layer "F.Cu") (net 2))
 (segment (start 185.837919 105.5) (end 187.825 105.5) (width 0.6) (layer "F.Cu") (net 7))
 (segment (start 182.54 108.797919) (end 185.837919 105.5) (width 0.6) (layer "F.Cu") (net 7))
 (segment (start 182.54 110) (end 182.54 108.797919) (width 0.6) (layer "F.Cu") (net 7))
 (segment (start 190.16 110) (end 193.39 106.77) (width 0.6) (layer "F.Cu") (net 1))
 (segment (start 193.39 106.77) (end 195 106.77) (width 0.6) (layer "F.Cu") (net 1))
 (segment (start 187.62 110) (end 190 112.38) (width 0.6) (layer "F.Cu") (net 3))
 (segment (start 193.3865 104.0125) (end 193.169 104.23) (width 0.6) (layer "F.Cu") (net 3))
 (segment (start 193.169 104.23) (end 195 104.23) (width 0.6) (layer "F.Cu") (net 3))
 (segment (start 190 112.38) (end 190 112.5) (width 0.6) (layer "F.Cu") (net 3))
 (segment (start 197.5 110.5) (end 197.5 105.820402) (width 0.6) (layer "F.Cu") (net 3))
 (segment (start 195.5 112.5) (end 197.5 110.5) (width 0.6) (layer "F.Cu") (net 3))
 (segment (start 197.5 105.820402) (end 195.909598 104.23) (width 0.6) (layer "F.Cu") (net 3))
 (segment (start 185 93) (end 193.3865 101.3865) (width 0.6) (layer "F.Cu") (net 3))
 (segment (start 195.909598 104.23) (end 195 104.23) (width 0.6) (layer "F.Cu") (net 3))
 (segment (start 190 112.5) (end 195.5 112.5) (width 0.6) (layer "F.Cu") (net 3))
 (segment (start 193.3865 101.3865) (end 193.3865 104.0125) (width 0.6) (layer "F.Cu") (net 3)))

